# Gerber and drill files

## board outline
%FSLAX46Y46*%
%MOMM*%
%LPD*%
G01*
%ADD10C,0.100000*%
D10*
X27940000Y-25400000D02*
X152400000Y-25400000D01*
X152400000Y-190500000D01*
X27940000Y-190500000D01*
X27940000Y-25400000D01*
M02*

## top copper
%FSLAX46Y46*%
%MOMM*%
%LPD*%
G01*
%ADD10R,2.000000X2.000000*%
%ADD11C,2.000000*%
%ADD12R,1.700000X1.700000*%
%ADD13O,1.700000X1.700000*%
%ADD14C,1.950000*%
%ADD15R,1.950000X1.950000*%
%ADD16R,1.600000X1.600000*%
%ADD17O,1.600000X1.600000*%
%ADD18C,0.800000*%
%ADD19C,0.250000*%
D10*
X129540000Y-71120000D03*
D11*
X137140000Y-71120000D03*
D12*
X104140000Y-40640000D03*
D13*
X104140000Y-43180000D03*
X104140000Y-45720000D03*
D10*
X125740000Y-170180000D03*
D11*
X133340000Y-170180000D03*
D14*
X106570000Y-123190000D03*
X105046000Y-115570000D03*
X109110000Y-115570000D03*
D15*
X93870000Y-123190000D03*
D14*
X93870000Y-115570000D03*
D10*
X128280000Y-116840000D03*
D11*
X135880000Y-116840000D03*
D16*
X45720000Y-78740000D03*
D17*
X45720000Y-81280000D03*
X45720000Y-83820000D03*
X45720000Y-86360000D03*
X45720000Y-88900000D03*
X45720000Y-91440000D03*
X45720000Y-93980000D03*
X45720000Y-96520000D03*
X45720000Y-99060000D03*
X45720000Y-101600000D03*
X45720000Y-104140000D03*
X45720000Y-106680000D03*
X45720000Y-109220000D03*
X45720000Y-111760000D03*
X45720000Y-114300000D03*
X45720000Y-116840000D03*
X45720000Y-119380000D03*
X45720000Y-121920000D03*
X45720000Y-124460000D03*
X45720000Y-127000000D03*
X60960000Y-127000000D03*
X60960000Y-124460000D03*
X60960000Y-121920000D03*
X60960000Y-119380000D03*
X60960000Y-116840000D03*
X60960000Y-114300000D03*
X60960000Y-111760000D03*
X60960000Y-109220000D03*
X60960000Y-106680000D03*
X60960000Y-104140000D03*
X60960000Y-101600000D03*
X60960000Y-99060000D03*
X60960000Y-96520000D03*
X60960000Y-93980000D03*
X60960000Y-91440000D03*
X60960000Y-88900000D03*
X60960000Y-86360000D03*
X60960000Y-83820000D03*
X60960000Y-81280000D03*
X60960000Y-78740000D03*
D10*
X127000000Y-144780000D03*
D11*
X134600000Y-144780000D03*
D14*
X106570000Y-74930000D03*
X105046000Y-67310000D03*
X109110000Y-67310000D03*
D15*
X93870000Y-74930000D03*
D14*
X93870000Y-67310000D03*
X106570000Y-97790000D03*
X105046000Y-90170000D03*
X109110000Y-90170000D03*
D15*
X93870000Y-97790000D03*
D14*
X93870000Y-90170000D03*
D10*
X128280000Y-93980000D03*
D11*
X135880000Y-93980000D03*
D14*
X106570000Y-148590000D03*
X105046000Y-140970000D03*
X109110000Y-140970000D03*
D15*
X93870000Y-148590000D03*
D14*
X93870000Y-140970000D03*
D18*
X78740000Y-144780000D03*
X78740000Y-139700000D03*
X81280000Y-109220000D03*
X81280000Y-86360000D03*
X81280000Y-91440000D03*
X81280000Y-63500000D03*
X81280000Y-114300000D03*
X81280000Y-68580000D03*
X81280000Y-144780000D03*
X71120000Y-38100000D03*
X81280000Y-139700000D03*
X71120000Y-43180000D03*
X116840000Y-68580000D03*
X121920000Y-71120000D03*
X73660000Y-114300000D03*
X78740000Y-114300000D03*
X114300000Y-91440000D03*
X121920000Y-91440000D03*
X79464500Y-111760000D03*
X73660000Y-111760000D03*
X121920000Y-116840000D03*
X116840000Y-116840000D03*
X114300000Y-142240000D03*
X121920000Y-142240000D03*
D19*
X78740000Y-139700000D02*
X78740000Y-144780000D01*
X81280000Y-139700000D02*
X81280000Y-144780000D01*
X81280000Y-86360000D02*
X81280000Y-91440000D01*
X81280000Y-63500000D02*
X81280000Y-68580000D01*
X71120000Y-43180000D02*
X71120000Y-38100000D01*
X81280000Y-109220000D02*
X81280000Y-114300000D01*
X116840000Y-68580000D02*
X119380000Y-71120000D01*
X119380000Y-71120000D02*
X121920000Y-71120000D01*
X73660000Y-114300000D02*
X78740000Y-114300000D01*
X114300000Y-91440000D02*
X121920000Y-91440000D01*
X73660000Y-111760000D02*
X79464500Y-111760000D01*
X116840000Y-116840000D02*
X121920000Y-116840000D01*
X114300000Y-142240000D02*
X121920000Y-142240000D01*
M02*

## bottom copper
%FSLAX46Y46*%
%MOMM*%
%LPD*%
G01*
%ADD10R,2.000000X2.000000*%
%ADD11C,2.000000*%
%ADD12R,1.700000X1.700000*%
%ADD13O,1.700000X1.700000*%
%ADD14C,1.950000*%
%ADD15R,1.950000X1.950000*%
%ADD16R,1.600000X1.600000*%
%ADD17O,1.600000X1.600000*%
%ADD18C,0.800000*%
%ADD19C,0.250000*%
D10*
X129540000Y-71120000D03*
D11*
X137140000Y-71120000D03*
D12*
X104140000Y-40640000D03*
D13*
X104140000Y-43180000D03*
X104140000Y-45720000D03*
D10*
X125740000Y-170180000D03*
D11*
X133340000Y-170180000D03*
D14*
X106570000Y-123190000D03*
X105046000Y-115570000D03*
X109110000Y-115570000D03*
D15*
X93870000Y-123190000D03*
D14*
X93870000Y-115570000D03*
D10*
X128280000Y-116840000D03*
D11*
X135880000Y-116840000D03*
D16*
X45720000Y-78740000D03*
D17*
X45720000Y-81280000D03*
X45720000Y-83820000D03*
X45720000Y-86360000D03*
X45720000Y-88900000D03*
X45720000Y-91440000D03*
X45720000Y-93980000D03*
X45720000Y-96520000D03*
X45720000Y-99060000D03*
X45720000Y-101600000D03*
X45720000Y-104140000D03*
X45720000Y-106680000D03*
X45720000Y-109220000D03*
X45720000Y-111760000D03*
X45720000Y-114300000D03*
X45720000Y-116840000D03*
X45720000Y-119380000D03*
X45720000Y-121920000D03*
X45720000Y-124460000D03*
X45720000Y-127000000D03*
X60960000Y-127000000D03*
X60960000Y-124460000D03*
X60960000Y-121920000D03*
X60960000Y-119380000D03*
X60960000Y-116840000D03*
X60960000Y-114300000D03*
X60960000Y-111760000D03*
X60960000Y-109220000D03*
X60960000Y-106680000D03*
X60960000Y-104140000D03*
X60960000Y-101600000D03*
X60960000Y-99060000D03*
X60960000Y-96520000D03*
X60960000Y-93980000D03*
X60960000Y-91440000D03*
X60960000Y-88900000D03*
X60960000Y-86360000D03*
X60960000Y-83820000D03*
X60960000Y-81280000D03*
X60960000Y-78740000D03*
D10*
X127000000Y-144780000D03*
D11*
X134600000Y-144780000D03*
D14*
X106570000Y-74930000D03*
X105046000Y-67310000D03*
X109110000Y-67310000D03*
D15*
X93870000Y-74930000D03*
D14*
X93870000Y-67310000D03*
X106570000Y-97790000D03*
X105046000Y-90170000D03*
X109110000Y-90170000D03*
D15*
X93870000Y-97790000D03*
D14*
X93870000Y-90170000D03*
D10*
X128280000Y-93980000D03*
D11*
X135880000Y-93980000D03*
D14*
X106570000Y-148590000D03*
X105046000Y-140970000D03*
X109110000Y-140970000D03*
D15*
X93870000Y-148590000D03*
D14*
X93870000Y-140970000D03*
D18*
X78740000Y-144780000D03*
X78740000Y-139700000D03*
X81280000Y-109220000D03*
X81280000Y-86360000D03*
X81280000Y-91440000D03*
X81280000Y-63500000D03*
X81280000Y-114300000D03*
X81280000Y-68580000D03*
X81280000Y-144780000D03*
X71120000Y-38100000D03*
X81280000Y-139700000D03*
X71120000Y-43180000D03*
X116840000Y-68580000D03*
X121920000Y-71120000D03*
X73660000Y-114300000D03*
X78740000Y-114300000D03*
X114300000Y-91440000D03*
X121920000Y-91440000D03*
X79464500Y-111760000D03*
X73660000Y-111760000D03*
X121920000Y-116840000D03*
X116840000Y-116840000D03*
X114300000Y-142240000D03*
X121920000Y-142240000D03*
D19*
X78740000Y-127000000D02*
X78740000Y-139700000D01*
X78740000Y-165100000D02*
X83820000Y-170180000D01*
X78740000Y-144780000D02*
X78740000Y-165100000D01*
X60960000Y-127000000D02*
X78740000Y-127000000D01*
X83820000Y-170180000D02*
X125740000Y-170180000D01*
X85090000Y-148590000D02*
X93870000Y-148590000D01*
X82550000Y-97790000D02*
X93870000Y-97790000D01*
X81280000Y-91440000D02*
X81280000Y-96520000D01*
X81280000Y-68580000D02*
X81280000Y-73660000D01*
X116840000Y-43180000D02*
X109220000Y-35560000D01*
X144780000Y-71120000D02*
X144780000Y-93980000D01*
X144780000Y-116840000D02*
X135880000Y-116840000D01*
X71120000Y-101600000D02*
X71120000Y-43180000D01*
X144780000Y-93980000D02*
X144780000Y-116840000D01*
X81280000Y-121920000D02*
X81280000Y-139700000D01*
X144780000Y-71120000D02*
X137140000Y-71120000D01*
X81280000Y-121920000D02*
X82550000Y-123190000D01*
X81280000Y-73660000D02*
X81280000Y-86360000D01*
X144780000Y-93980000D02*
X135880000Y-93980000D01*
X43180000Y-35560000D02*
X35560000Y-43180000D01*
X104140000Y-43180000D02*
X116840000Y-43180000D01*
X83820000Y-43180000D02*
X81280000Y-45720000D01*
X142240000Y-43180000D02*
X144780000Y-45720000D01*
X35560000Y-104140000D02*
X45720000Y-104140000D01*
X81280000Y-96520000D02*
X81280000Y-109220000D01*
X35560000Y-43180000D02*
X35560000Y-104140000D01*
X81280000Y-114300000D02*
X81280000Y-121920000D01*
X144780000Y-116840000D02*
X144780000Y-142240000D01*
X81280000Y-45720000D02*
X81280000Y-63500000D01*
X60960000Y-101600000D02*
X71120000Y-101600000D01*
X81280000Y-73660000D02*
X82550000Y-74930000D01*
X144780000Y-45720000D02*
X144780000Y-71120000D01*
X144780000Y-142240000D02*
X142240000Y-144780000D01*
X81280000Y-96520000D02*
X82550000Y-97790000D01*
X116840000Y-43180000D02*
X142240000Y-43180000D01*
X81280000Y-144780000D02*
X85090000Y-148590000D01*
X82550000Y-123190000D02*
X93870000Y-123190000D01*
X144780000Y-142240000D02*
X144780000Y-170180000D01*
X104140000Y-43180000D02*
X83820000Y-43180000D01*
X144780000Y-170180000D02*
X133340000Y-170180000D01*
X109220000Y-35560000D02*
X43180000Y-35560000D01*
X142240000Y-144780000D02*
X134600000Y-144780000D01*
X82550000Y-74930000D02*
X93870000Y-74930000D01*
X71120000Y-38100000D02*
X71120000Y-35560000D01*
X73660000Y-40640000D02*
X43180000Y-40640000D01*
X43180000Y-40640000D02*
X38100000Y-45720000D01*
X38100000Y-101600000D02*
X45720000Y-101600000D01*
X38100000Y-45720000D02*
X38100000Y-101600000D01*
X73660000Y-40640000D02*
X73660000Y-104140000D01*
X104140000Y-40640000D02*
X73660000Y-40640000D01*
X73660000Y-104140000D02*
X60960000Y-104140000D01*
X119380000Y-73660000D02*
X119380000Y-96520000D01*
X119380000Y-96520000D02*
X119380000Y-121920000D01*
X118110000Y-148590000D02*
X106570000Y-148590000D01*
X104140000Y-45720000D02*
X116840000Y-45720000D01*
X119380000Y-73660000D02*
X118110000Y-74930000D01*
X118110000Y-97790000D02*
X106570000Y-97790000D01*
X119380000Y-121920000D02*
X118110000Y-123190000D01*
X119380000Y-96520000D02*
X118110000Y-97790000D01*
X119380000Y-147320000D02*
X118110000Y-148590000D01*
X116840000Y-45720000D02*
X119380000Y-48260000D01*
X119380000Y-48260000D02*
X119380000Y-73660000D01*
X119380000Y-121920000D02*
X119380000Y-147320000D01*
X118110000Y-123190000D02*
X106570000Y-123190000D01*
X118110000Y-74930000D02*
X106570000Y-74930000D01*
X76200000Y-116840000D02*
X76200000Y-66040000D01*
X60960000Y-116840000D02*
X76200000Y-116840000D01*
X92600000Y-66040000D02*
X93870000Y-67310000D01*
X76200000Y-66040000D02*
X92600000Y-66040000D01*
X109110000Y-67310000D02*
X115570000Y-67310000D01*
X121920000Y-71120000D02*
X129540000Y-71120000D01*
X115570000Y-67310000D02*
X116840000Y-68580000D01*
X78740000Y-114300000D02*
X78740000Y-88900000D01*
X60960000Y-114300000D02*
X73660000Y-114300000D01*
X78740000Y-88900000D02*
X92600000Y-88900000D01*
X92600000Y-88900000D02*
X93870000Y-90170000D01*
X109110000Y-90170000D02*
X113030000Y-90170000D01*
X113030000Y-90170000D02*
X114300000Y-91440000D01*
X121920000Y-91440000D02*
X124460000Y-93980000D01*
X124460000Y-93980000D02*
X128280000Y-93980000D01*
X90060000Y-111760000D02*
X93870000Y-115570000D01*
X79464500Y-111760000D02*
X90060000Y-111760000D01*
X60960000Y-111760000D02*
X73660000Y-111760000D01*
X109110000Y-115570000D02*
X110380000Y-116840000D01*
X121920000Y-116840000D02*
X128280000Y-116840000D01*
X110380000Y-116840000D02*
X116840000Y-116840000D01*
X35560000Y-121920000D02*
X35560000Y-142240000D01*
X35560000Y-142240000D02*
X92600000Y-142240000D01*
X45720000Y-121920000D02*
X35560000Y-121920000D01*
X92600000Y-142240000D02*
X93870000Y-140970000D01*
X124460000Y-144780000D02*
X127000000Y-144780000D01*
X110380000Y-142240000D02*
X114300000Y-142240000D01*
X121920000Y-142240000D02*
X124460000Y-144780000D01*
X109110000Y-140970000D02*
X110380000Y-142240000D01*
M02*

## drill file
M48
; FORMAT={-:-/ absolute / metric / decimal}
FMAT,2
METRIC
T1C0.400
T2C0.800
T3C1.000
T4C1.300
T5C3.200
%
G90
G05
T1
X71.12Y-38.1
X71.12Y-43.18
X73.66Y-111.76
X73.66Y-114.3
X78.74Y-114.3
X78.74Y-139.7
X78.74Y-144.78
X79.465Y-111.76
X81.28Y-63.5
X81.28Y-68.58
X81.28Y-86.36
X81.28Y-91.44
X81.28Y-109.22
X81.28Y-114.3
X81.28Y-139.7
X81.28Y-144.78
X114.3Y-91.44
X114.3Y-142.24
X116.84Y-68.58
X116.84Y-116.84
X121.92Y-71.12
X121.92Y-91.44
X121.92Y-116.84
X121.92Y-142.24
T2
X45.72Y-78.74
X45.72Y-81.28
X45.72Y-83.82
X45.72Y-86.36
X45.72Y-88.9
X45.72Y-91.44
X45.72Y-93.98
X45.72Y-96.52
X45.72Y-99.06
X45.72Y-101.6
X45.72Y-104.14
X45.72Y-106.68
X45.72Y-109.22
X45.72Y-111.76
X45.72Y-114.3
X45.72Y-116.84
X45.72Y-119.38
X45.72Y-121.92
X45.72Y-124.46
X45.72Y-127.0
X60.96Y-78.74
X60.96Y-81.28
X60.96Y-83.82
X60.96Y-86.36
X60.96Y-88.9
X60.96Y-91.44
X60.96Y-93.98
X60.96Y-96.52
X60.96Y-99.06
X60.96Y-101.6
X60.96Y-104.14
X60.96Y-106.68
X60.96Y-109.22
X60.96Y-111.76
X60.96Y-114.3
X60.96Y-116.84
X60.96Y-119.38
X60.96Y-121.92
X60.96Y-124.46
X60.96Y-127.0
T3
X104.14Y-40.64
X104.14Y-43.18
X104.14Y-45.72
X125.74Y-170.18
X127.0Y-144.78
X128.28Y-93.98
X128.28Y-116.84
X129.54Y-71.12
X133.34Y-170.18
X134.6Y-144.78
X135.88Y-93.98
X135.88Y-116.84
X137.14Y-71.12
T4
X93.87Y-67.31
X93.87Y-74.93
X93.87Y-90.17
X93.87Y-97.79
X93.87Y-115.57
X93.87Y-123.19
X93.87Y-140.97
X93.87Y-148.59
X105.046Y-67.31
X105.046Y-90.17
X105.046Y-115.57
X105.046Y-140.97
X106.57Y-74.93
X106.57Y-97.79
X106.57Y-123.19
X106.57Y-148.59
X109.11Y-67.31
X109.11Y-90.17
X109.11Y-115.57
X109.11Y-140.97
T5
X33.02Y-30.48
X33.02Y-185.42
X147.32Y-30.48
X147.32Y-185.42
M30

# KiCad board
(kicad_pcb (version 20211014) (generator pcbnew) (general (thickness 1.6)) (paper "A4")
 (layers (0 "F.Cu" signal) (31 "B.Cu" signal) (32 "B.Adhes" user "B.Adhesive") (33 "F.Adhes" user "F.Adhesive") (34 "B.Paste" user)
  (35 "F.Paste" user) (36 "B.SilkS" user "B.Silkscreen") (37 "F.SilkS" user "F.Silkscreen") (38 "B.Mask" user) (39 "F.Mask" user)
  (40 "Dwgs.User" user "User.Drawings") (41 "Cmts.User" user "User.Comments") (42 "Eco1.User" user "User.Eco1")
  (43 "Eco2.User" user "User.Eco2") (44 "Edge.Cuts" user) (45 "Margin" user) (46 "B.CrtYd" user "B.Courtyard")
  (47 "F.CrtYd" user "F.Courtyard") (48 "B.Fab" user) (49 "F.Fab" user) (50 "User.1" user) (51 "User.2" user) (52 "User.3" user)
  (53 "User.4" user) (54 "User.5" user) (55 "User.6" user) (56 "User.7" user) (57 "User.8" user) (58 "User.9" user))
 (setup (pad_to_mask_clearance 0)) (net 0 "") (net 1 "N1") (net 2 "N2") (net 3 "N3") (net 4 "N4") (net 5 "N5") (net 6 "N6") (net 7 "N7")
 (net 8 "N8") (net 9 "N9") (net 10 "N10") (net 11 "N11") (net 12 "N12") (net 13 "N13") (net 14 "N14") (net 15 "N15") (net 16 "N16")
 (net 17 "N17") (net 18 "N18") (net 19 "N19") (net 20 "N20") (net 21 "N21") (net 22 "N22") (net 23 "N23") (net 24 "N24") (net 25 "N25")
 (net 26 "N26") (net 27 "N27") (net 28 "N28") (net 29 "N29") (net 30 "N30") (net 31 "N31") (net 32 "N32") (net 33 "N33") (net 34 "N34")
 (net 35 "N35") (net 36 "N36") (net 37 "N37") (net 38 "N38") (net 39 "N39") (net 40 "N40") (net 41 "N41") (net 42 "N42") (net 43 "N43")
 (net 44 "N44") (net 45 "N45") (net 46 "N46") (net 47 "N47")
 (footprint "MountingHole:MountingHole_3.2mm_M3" (layer "F.Cu") (at 33.02 30.48)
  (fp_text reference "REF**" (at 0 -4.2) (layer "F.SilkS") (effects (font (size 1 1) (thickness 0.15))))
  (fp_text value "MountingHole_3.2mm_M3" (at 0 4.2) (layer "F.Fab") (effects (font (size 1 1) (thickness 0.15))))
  (pad "" np_thru_hole circle (at 0 0) (size 3.2 3.2) (drill 3.2) (layers *.Cu *.Mask)))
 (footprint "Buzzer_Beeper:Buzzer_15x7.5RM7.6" (layer "F.Cu") (at 129.54 71.12)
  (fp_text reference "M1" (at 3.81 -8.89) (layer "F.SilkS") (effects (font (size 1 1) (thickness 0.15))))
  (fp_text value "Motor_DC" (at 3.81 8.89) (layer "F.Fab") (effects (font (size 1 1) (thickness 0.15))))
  (pad "1" thru_hole rect (at 0 0) (size 2 2) (drill 1) (layers *.Cu *.Mask) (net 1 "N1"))
  (pad "2" thru_hole circle (at 7.6 0) (size 2 2) (drill 1) (layers *.Cu *.Mask) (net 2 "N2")))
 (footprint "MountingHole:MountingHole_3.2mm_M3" (layer "F.Cu") (at 33.02 185.42)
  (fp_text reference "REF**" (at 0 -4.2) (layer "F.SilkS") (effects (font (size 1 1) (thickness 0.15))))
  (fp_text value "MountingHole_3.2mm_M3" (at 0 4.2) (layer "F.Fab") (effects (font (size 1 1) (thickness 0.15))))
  (pad "" np_thru_hole circle (at 0 0) (size 3.2 3.2) (drill 3.2) (layers *.Cu *.Mask)))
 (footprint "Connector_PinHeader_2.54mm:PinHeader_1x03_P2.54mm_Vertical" (layer "F.Cu") (at 104.14 40.64)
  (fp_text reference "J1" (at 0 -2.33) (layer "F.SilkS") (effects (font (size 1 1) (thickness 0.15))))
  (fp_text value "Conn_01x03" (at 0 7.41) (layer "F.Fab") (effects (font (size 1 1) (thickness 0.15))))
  (pad "1" thru_hole rect (at 0 0) (size 1.7 1.7) (drill 1) (layers *.Cu *.Mask) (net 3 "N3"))
  (pad "2" thru_hole oval (at 0 2.54) (size 1.7 1.7) (drill 1) (layers *.Cu *.Mask) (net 2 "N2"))
  (pad "3" thru_hole oval (at 0 5.08) (size 1.7 1.7) (drill 1) (layers *.Cu *.Mask) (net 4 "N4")))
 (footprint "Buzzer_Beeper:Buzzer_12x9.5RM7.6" (layer "F.Cu") (at 125.74 170.18)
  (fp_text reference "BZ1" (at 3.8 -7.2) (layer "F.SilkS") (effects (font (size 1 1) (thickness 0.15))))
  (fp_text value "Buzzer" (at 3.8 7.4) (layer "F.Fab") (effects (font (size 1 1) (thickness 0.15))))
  (pad "1" thru_hole rect (at 0 0) (size 2 2) (drill 1) (layers *.Cu *.Mask) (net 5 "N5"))
  (pad "2" thru_hole circle (at 7.6 0) (size 2 2) (drill 1) (layers *.Cu *.Mask) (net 2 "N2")))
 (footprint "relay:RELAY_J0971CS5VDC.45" (layer "F.Cu") (at 101.6 119.38)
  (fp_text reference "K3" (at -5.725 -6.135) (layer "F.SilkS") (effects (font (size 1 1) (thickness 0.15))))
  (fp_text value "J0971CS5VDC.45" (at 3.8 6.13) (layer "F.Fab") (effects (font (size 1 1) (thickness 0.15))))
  (pad "11" thru_hole circle locked (at 4.97 3.81) (size 1.95 1.95) (drill 1.3) (layers *.Cu *.Mask) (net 4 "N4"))
  (pad "12" thru_hole circle locked (at 3.446 -3.81) (size 1.95 1.95) (drill 1.3) (layers *.Cu *.Mask) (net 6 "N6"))
  (pad "14" thru_hole circle locked (at 7.51 -3.81) (size 1.95 1.95) (drill 1.3) (layers *.Cu *.Mask) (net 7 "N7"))
  (pad "A1" thru_hole rect locked (at -7.73 3.81) (size 1.95 1.95) (drill 1.3) (layers *.Cu *.Mask) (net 2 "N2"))
  (pad "A2" thru_hole circle locked (at -7.73 -3.81) (size 1.95 1.95) (drill 1.3) (layers *.Cu *.Mask) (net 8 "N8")))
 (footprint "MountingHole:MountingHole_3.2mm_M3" (layer "F.Cu") (at 147.32 30.48)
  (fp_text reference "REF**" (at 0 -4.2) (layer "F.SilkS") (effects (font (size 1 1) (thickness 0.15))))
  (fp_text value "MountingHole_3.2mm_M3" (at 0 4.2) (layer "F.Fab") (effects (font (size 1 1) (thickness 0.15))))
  (pad "" np_thru_hole circle (at 0 0) (size 3.2 3.2) (drill 3.2) (layers *.Cu *.Mask)))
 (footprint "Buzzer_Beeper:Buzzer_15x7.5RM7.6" (layer "F.Cu") (at 128.28 116.84)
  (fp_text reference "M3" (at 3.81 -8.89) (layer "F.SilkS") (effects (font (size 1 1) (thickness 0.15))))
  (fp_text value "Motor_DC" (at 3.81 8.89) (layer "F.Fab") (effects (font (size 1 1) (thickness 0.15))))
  (pad "1" thru_hole rect (at 0 0) (size 2 2) (drill 1) (layers *.Cu *.Mask) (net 7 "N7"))
  (pad "2" thru_hole circle (at 7.6 0) (size 2 2) (drill 1) (layers *.Cu *.Mask) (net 2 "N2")))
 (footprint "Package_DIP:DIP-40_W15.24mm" (layer "F.Cu") (at 45.72 78.74)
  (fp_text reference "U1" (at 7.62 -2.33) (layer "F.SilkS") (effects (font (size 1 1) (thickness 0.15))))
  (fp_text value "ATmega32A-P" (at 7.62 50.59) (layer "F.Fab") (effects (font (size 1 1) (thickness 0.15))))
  (pad "1" thru_hole rect (at 0 0) (size 1.6 1.6) (drill 0.8) (layers *.Cu *.Mask) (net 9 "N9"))
  (pad "2" thru_hole oval (at 0 2.54) (size 1.6 1.6) (drill 0.8) (layers *.Cu *.Mask) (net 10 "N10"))
  (pad "3" thru_hole oval (at 0 5.08) (size 1.6 1.6) (drill 0.8) (layers *.Cu *.Mask) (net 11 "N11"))
  (pad "4" thru_hole oval (at 0 7.62) (size 1.6 1.6) (drill 0.8) (layers *.Cu *.Mask) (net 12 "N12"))
  (pad "5" thru_hole oval (at 0 10.16) (size 1.6 1.6) (drill 0.8) (layers *.Cu *.Mask) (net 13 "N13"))
  (pad "6" thru_hole oval (at 0 12.7) (size 1.6 1.6) (drill 0.8) (layers *.Cu *.Mask) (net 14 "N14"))
  (pad "7" thru_hole oval (at 0 15.24) (size 1.6 1.6) (drill 0.8) (layers *.Cu *.Mask) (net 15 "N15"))
  (pad "8" thru_hole oval (at 0 17.78) (size 1.6 1.6) (drill 0.8) (layers *.Cu *.Mask) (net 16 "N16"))
  (pad "9" thru_hole oval (at 0 20.32) (size 1.6 1.6) (drill 0.8) (layers *.Cu *.Mask) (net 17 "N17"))
  (pad "10" thru_hole oval (at 0 22.86) (size 1.6 1.6) (drill 0.8) (layers *.Cu *.Mask) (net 3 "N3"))
  (pad "11" thru_hole oval (at 0 25.4) (size 1.6 1.6) (drill 0.8) (layers *.Cu *.Mask) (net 2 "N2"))
  (pad "12" thru_hole oval (at 0 27.94) (size 1.6 1.6) (drill 0.8) (layers *.Cu *.Mask) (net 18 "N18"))
  (pad "13" thru_hole oval (at 0 30.48) (size 1.6 1.6) (drill 0.8) (layers *.Cu *.Mask) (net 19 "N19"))
  (pad "14" thru_hole oval (at 0 33.02) (size 1.6 1.6) (drill 0.8) (layers *.Cu *.Mask) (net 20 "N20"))
  (pad "15" thru_hole oval (at 0 35.56) (size 1.6 1.6) (drill 0.8) (layers *.Cu *.Mask) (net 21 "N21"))
  (pad "16" thru_hole oval (at 0 38.1) (size 1.6 1.6) (drill 0.8) (layers *.Cu *.Mask) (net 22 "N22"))
  (pad "17" thru_hole oval (at 0 40.64) (size 1.6 1.6) (drill 0.8) (layers *.Cu *.Mask) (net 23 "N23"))
  (pad "18" thru_hole oval (at 0 43.18) (size 1.6 1.6) (drill 0.8) (layers *.Cu *.Mask) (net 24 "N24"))
  (pad "19" thru_hole oval (at 0 45.72) (size 1.6 1.6) (drill 0.8) (layers *.Cu *.Mask) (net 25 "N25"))
  (pad "20" thru_hole oval (at 0 48.26) (size 1.6 1.6) (drill 0.8) (layers *.Cu *.Mask) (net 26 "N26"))
  (pad "21" thru_hole oval (at 15.24 48.26) (size 1.6 1.6) (drill 0.8) (layers *.Cu *.Mask) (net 5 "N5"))
  (pad "22" thru_hole oval (at 15.24 45.72) (size 1.6 1.6) (drill 0.8) (layers *.Cu *.Mask) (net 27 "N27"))
  (pad "23" thru_hole oval (at 15.24 43.18) (size 1.6 1.6) (drill 0.8) (layers *.Cu *.Mask) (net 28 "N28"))
  (pad "24" thru_hole oval (at 15.24 40.64) (size 1.6 1.6) (drill 0.8) (layers *.Cu *.Mask) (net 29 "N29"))
  (pad "25" thru_hole oval (at 15.24 38.1) (size 1.6 1.6) (drill 0.8) (layers *.Cu *.Mask) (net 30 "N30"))
  (pad "26" thru_hole oval (at 15.24 35.56) (size 1.6 1.6) (drill 0.8) (layers *.Cu *.Mask) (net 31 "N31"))
  (pad "27" thru_hole oval (at 15.24 33.02) (size 1.6 1.6) (drill 0.8) (layers *.Cu *.Mask) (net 8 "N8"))
  (pad "28" thru_hole oval (at 15.24 30.48) (size 1.6 1.6) (drill 0.8) (layers *.Cu *.Mask) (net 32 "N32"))
  (pad "29" thru_hole oval (at 15.24 27.94) (size 1.6 1.6) (drill 0.8) (layers *.Cu *.Mask) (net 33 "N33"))
  (pad "30" thru_hole oval (at 15.24 25.4) (size 1.6 1.6) (drill 0.8) (layers *.Cu *.Mask) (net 3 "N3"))
  (pad "31" thru_hole oval (at 15.24 22.86) (size 1.6 1.6) (drill 0.8) (layers *.Cu *.Mask) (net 2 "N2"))
  (pad "32" thru_hole oval (at 15.24 20.32) (size 1.6 1.6) (drill 0.8) (layers *.Cu *.Mask) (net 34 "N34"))
  (pad "33" thru_hole oval (at 15.24 17.78) (size 1.6 1.6) (drill 0.8) (layers *.Cu *.Mask) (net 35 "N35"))
  (pad "34" thru_hole oval (at 15.24 15.24) (size 1.6 1.6) (drill 0.8) (layers *.Cu *.Mask) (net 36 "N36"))
  (pad "35" thru_hole oval (at 15.24 12.7) (size 1.6 1.6) (drill 0.8) (layers *.Cu *.Mask) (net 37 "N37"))
  (pad "36" thru_hole oval (at 15.24 10.16) (size 1.6 1.6) (drill 0.8) (layers *.Cu *.Mask) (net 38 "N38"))
  (pad "37" thru_hole oval (at 15.24 7.62) (size 1.6 1.6) (drill 0.8) (layers *.Cu *.Mask) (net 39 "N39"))
  (pad "38" thru_hole oval (at 15.24 5.08) (size 1.6 1.6) (drill 0.8) (layers *.Cu *.Mask) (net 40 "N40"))
  (pad "39" thru_hole oval (at 15.24 2.54) (size 1.6 1.6) (drill 0.8) (layers *.Cu *.Mask) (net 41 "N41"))
  (pad "40" thru_hole oval (at 15.24 0) (size 1.6 1.6) (drill 0.8) (layers *.Cu *.Mask) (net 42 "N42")))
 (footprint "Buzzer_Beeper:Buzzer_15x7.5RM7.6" (layer "F.Cu") (at 127 144.78)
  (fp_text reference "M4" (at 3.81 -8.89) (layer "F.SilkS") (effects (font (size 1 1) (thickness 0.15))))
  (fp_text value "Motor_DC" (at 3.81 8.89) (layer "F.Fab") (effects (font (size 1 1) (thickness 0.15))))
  (pad "1" thru_hole rect (at 0 0) (size 2 2) (drill 1) (layers *.Cu *.Mask) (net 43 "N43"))
  (pad "2" thru_hole circle (at 7.6 0) (size 2 2) (drill 1) (layers *.Cu *.Mask) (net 2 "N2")))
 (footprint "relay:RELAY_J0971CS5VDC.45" (layer "F.Cu") (at 101.6 71.12)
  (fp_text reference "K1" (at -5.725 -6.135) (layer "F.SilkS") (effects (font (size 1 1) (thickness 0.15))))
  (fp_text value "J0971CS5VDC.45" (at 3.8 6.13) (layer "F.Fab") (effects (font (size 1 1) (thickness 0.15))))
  (pad "11" thru_hole circle locked (at 4.97 3.81) (size 1.95 1.95) (drill 1.3) (layers *.Cu *.Mask) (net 4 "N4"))
  (pad "12" thru_hole circle locked (at 3.446 -3.81) (size 1.95 1.95) (drill 1.3) (layers *.Cu *.Mask) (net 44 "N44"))
  (pad "14" thru_hole circle locked (at 7.51 -3.81) (size 1.95 1.95) (drill 1.3) (layers *.Cu *.Mask) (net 1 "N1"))
  (pad "A1" thru_hole rect locked (at -7.73 3.81) (size 1.95 1.95) (drill 1.3) (layers *.Cu *.Mask) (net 2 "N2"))
  (pad "A2" thru_hole circle locked (at -7.73 -3.81) (size 1.95 1.95) (drill 1.3) (layers *.Cu *.Mask) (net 30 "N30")))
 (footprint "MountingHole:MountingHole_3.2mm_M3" (layer "F.Cu") (at 147.32 185.42)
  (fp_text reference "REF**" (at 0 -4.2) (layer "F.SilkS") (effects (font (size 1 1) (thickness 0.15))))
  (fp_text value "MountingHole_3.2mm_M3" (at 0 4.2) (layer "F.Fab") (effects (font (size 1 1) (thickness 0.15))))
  (pad "" np_thru_hole circle (at 0 0) (size 3.2 3.2) (drill 3.2) (layers *.Cu *.Mask)))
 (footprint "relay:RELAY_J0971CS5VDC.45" (layer "F.Cu") (at 101.6 93.98)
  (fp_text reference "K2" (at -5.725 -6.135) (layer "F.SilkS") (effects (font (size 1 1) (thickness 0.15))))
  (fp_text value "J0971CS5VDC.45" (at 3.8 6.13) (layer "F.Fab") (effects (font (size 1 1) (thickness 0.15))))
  (pad "11" thru_hole circle locked (at 4.97 3.81) (size 1.95 1.95) (drill 1.3) (layers *.Cu *.Mask) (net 4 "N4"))
  (pad "12" thru_hole circle locked (at 3.446 -3.81) (size 1.95 1.95) (drill 1.3) (layers *.Cu *.Mask) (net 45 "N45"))
  (pad "14" thru_hole circle locked (at 7.51 -3.81) (size 1.95 1.95) (drill 1.3) (layers *.Cu *.Mask) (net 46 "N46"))
  (pad "A1" thru_hole rect locked (at -7.73 3.81) (size 1.95 1.95) (drill 1.3) (layers *.Cu *.Mask) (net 2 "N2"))
  (pad "A2" thru_hole circle locked (at -7.73 -3.81) (size 1.95 1.95) (drill 1.3) (layers *.Cu *.Mask) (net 31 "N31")))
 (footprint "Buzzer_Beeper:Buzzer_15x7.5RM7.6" (layer "F.Cu") (at 128.28 93.98)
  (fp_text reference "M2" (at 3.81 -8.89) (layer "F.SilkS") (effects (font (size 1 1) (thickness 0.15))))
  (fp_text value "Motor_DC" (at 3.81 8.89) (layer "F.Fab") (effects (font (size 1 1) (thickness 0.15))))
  (pad "1" thru_hole rect (at 0 0) (size 2 2) (drill 1) (layers *.Cu *.Mask) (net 46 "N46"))
  (pad "2" thru_hole circle (at 7.6 0) (size 2 2) (drill 1) (layers *.Cu *.Mask) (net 2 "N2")))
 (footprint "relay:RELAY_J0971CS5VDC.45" (layer "F.Cu") (at 101.6 144.78)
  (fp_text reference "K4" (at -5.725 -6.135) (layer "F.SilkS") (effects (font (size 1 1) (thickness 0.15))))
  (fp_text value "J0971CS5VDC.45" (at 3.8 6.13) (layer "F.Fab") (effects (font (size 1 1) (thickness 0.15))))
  (pad "11" thru_hole circle locked (at 4.97 3.81) (size 1.95 1.95) (drill 1.3) (layers *.Cu *.Mask) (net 4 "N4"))
  (pad "12" thru_hole circle locked (at 3.446 -3.81) (size 1.95 1.95) (drill 1.3) (layers *.Cu *.Mask) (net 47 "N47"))
  (pad "14" thru_hole circle locked (at 7.51 -3.81) (size 1.95 1.95) (drill 1.3) (layers *.Cu *.Mask) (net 43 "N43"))
  (pad "A1" thru_hole rect locked (at -7.73 3.81) (size 1.95 1.95) (drill 1.3) (layers *.Cu *.Mask) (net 2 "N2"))
  (pad "A2" thru_hole circle locked (at -7.73 -3.81) (size 1.95 1.95) (drill 1.3) (layers *.Cu *.Mask) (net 24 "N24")))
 (gr_rect (start 27.94 25.4) (end 152.4 190.5) (layer "Edge.Cuts") (width 0.1) (fill none))
 (segment (start 78.74 139.7) (end 78.74 144.78) (width 0.25) (layer "F.Cu") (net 5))
 (via (at 78.74 144.78) (size 0.8) (drill 0.4) (layers "F.Cu" "B.Cu") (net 5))
 (via (at 78.74 139.7) (size 0.8) (drill 0.4) (layers "F.Cu" "B.Cu") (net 5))
 (segment (start 78.74 127) (end 78.74 139.7) (width 0.25) (layer "B.Cu") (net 5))
 (segment (start 78.74 165.1) (end 83.82 170.18) (width 0.25) (layer "B.Cu") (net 5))
 (segment (start 78.74 144.78) (end 78.74 165.1) (width 0.25) (layer "B.Cu") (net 5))
 (segment (start 60.96 127) (end 78.74 127) (width 0.25) (layer "B.Cu") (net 5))
 (segment (start 83.82 170.18) (end 125.74 170.18) (width 0.25) (layer "B.Cu") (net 5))
 (segment (start 81.28 139.7) (end 81.28 144.78) (width 0.25) (layer "F.Cu") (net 2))
 (segment (start 81.28 86.36) (end 81.28 91.44) (width 0.25) (layer "F.Cu") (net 2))
 (segment (start 81.28 63.5) (end 81.28 68.58) (width 0.25) (layer "F.Cu") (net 2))
 (segment (start 71.12 43.18) (end 71.12 38.1) (width 0.25) (layer "F.Cu") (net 2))
 (segment (start 81.28 109.22) (end 81.28 114.3) (width 0.25) (layer "F.Cu") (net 2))
 (via (at 81.28 109.22) (size 0.8) (drill 0.4) (layers "F.Cu" "B.Cu") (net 2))
 (via (at 81.28 86.36) (size 0.8) (drill 0.4) (layers "F.Cu" "B.Cu") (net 2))
 (via (at 81.28 91.44) (size 0.8) (drill 0.4) (layers "F.Cu" "B.Cu") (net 2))
 (via (at 81.28 63.5) (size 0.8) (drill 0.4) (layers "F.Cu" "B.Cu") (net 2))
 (via (at 81.28 114.3) (size 0.8) (drill 0.4) (layers "F.Cu" "B.Cu") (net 2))
 (via (at 81.28 68.58) (size 0.8) (drill 0.4) (layers "F.Cu" "B.Cu") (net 2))
 (via (at 81.28 144.78) (size 0.8) (drill 0.4) (layers "F.Cu" "B.Cu") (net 2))
 (via (at 71.12 38.1) (size 0.8) (drill 0.4) (layers "F.Cu" "B.Cu") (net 2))
 (via (at 81.28 139.7) (size 0.8) (drill 0.4) (layers "F.Cu" "B.Cu") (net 2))
 (via (at 71.12 43.18) (size 0.8) (drill 0.4) (layers "F.Cu" "B.Cu") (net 2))
 (segment (start 85.09 148.59) (end 93.87 148.59) (width 0.25) (layer "B.Cu") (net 2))
 (segment (start 82.55 97.79) (end 93.87 97.79) (width 0.25) (layer "B.Cu") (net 2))
 (segment (start 81.28 91.44) (end 81.28 96.52) (width 0.25) (layer "B.Cu") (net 2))
 (segment (start 81.28 68.58) (end 81.28 73.66) (width 0.25) (layer "B.Cu") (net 2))
 (segment (start 116.84 43.18) (end 109.22 35.56) (width 0.25) (layer "B.Cu") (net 2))
 (segment (start 144.78 71.12) (end 144.78 93.98) (width 0.25) (layer "B.Cu") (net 2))
 (segment (start 144.78 116.84) (end 135.88 116.84) (width 0.25) (layer "B.Cu") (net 2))
 (segment (start 71.12 101.6) (end 71.12 43.18) (width 0.25) (layer "B.Cu") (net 2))
 (segment (start 144.78 93.98) (end 144.78 116.84) (width 0.25) (layer "B.Cu") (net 2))
 (segment (start 81.28 121.92) (end 81.28 139.7) (width 0.25) (layer "B.Cu") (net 2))
 (segment (start 144.78 71.12) (end 137.14 71.12) (width 0.25) (layer "B.Cu") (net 2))
 (segment (start 81.28 121.92) (end 82.55 123.19) (width 0.25) (layer "B.Cu") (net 2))
 (segment (start 81.28 73.66) (end 81.28 86.36) (width 0.25) (layer "B.Cu") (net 2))
 (segment (start 144.78 93.98) (end 135.88 93.98) (width 0.25) (layer "B.Cu") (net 2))
 (segment (start 43.18 35.56) (end 35.56 43.18) (width 0.25) (layer "B.Cu") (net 2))
 (segment (start 104.14 43.18) (end 116.84 43.18) (width 0.25) (layer "B.Cu") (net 2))
 (segment (start 83.82 43.18) (end 81.28 45.72) (width 0.25) (layer "B.Cu") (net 2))
 (segment (start 142.24 43.18) (end 144.78 45.72) (width 0.25) (layer "B.Cu") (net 2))
 (segment (start 35.56 104.14) (end 45.72 104.14) (width 0.25) (layer "B.Cu") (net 2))
 (segment (start 81.28 96.52) (end 81.28 109.22) (width 0.25) (layer "B.Cu") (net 2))
 (segment (start 35.56 43.18) (end 35.56 104.14) (width 0.25) (layer "B.Cu") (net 2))
 (segment (start 81.28 114.3) (end 81.28 121.92) (width 0.25) (layer "B.Cu") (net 2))
 (segment (start 144.78 116.84) (end 144.78 142.24) (width 0.25) (layer "B.Cu") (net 2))
 (segment (start 81.28 45.72) (end 81.28 63.5) (width 0.25) (layer "B.Cu") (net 2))
 (segment (start 60.96 101.6) (end 71.12 101.6) (width 0.25) (layer "B.Cu") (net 2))
 (segment (start 81.28 73.66) (end 82.55 74.93) (width 0.25) (layer "B.Cu") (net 2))
 (segment (start 144.78 45.72) (end 144.78 71.12) (width 0.25) (layer "B.Cu") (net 2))
 (segment (start 144.78 142.24) (end 142.24 144.78) (width 0.25) (layer "B.Cu") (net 2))
 (segment (start 81.28 96.52) (end 82.55 97.79) (width 0.25) (layer "B.Cu") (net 2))
 (segment (start 116.84 43.18) (end 142.24 43.18) (width 0.25) (layer "B.Cu") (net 2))
 (segment (start 81.28 144.78) (end 85.09 148.59) (width 0.25) (layer "B.Cu") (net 2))
 (segment (start 82.55 123.19) (end 93.87 123.19) (width 0.25) (layer "B.Cu") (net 2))
 (segment (start 144.78 142.24) (end 144.78 170.18) (width 0.25) (layer "B.Cu") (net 2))
 (segment (start 104.14 43.18) (end 83.82 43.18) (width 0.25) (layer "B.Cu") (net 2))
 (segment (start 144.78 170.18) (end 133.34 170.18) (width 0.25) (layer "B.Cu") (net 2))
 (segment (start 109.22 35.56) (end 43.18 35.56) (width 0.25) (layer "B.Cu") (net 2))
 (segment (start 142.24 144.78) (end 134.6 144.78) (width 0.25) (layer "B.Cu") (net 2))
 (segment (start 82.55 74.93) (end 93.87 74.93) (width 0.25) (layer "B.Cu") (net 2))
 (segment (start 71.12 38.1) (end 71.12 35.56) (width 0.25) (layer "B.Cu") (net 2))
 (segment (start 73.66 40.64) (end 43.18 40.64) (width 0.25) (layer "B.Cu") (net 3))
 (segment (start 43.18 40.64) (end 38.1 45.72) (width 0.25) (layer "B.Cu") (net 3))
 (segment (start 38.1 101.6) (end 45.72 101.6) (width 0.25) (layer "B.Cu") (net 3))
 (segment (start 38.1 45.72) (end 38.1 101.6) (width 0.25) (layer "B.Cu") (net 3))
 (segment (start 73.66 40.64) (end 73.66 104.14) (width 0.25) (layer "B.Cu") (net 3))
 (segment (start 104.14 40.64) (end 73.66 40.64) (width 0.25) (layer "B.Cu") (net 3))
 (segment (start 73.66 104.14) (end 60.96 104.14) (width 0.25) (layer "B.Cu") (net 3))
 (segment (start 119.38 73.66) (end 119.38 96.52) (width 0.25) (layer "B.Cu") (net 4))
 (segment (start 119.38 96.52) (end 119.38 121.92) (width 0.25) (layer "B.Cu") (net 4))
 (segment (start 118.11 148.59) (end 106.57 148.59) (width 0.25) (layer "B.Cu") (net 4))
 (segment (start 104.14 45.72) (end 116.84 45.72) (width 0.25) (layer "B.Cu") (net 4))
 (segment (start 119.38 73.66) (end 118.11 74.93) (width 0.25) (layer "B.Cu") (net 4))
 (segment (start 118.11 97.79) (end 106.57 97.79) (width 0.25) (layer "B.Cu") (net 4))
 (segment (start 119.38 121.92) (end 118.11 123.19) (width 0.25) (layer "B.Cu") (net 4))
 (segment (start 119.38 96.52) (end 118.11 97.79) (width 0.25) (layer "B.Cu") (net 4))
 (segment (start 119.38 147.32) (end 118.11 148.59) (width 0.25) (layer "B.Cu") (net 4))
 (segment (start 116.84 45.72) (end 119.38 48.26) (width 0.25) (layer "B.Cu") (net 4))
 (segment (start 119.38 48.26) (end 119.38 73.66) (width 0.25) (layer "B.Cu") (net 4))
 (segment (start 119.38 121.92) (end 119.38 147.32) (width 0.25) (layer "B.Cu") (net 4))
 (segment (start 118.11 123.19) (end 106.57 123.19) (width 0.25) (layer "B.Cu") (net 4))
 (segment (start 118.11 74.93) (end 106.57 74.93) (width 0.25) (layer "B.Cu") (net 4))
 (segment (start 76.2 116.84) (end 76.2 66.04) (width 0.25) (layer "B.Cu") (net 30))
 (segment (start 60.96 116.84) (end 76.2 116.84) (width 0.25) (layer "B.Cu") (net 30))
 (segment (start 92.6 66.04) (end 93.87 67.31) (width 0.25) (layer "B.Cu") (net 30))
 (segment (start 76.2 66.04) (end 92.6 66.04) (width 0.25) (layer "B.Cu") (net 30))
 (segment (start 116.84 68.58) (end 119.38 71.12) (width 0.25) (layer "F.Cu") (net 1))
 (segment (start 119.38 71.12) (end 121.92 71.12) (width 0.25) (layer "F.Cu") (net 1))
 (via (at 116.84 68.58) (size 0.8) (drill 0.4) (layers "F.Cu" "B.Cu") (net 1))
 (via (at 121.92 71.12) (size 0.8) (drill 0.4) (layers "F.Cu" "B.Cu") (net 1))
 (segment (start 109.11 67.31) (end 115.57 67.31) (width 0.25) (layer "B.Cu") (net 1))
 (segment (start 121.92 71.12) (end 129.54 71.12) (width 0.25) (layer "B.Cu") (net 1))
 (segment (start 115.57 67.31) (end 116.84 68.58) (width 0.25) (layer "B.Cu") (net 1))
 (segment (start 73.66 114.3) (end 78.74 114.3) (width 0.25) (layer "F.Cu") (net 31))
 (via (at 73.66 114.3) (size 0.8) (drill 0.4) (layers "F.Cu" "B.Cu") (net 31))
 (via (at 78.74 114.3) (size 0.8) (drill 0.4) (layers "F.Cu" "B.Cu") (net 31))
 (segment (start 78.74 114.3) (end 78.74 88.9) (width 0.25) (layer "B.Cu") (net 31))
 (segment (start 60.96 114.3) (end 73.66 114.3) (width 0.25) (layer "B.Cu") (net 31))
 (segment (start 78.74 88.9) (end 92.6 88.9) (width 0.25) (layer "B.Cu") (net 31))
 (segment (start 92.6 88.9) (end 93.87 90.17) (width 0.25) (layer "B.Cu") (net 31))
 (segment (start 114.3 91.44) (end 121.92 91.44) (width 0.25) (layer "F.Cu") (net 46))
 (via (at 114.3 91.44) (size 0.8) (drill 0.4) (layers "F.Cu" "B.Cu") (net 46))
 (via (at 121.92 91.44) (size 0.8) (drill 0.4) (layers "F.Cu" "B.Cu") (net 46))
 (segment (start 109.11 90.17) (end 113.03 90.17) (width 0.25) (layer "B.Cu") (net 46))
 (segment (start 113.03 90.17) (end 114.3 91.44) (width 0.25) (layer "B.Cu") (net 46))
 (segment (start 121.92 91.44) (end 124.46 93.98) (width 0.25) (layer "B.Cu") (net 46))
 (segment (start 124.46 93.98) (end 128.28 93.98) (width 0.25) (layer "B.Cu") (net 46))
 (segment (start 73.66 111.76) (end 79.4645 111.76) (width 0.25) (layer "F.Cu") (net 8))
 (via (at 79.4645 111.76) (size 0.8) (drill 0.4) (layers "F.Cu" "B.Cu") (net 8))
 (via (at 73.66 111.76) (size 0.8) (drill 0.4) (layers "F.Cu" "B.Cu") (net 8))
 (segment (start 90.06 111.76) (end 93.87 115.57) (width 0.25) (layer "B.Cu") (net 8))
 (segment (start 79.4645 111.76) (end 90.06 111.76) (width 0.25) (layer "B.Cu") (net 8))
 (segment (start 60.96 111.76) (end 73.66 111.76) (width 0.25) (layer "B.Cu") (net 8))
 (segment (start 116.84 116.84) (end 121.92 116.84) (width 0.25) (layer "F.Cu") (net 7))
 (via (at 121.92 116.84) (size 0.8) (drill 0.4) (layers "F.Cu" "B.Cu") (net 7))
 (via (at 116.84 116.84) (size 0.8) (drill 0.4) (layers "F.Cu" "B.Cu") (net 7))
 (segment (start 109.11 115.57) (end 110.38 116.84) (width 0.25) (layer "B.Cu") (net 7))
 (segment (start 121.92 116.84) (end 128.28 116.84) (width 0.25) (layer "B.Cu") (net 7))
 (segment (start 110.38 116.84) (end 116.84 116.84) (width 0.25) (layer "B.Cu") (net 7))
 (segment (start 35.56 121.92) (end 35.56 142.24) (width 0.25) (layer "B.Cu") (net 24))
 (segment (start 35.56 142.24) (end 92.6 142.24) (width 0.25) (layer "B.Cu") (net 24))
 (segment (start 45.72 121.92) (end 35.56 121.92) (width 0.25) (layer "B.Cu") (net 24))
 (segment (start 92.6 142.24) (end 93.87 140.97) (width 0.25) (layer "B.Cu") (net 24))
 (segment (start 114.3 142.24) (end 121.92 142.24) (width 0.25) (layer "F.Cu") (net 43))
 (via (at 114.3 142.24) (size 0.8) (drill 0.4) (layers "F.Cu" "B.Cu") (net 43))
 (via (at 121.92 142.24) (size 0.8) (drill 0.4) (layers "F.Cu" "B.Cu") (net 43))
 (segment (start 124.46 144.78) (end 127 144.78) (width 0.25) (layer "B.Cu") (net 43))
 (segment (start 110.38 142.24) (end 114.3 142.24) (width 0.25) (layer "B.Cu") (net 43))
 (segment (start 121.92 142.24) (end 124.46 144.78) (width 0.25) (layer "B.Cu") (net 43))
 (segment (start 109.11 140.97) (end 110.38 142.24) (width 0.25) (layer "B.Cu") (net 43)))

